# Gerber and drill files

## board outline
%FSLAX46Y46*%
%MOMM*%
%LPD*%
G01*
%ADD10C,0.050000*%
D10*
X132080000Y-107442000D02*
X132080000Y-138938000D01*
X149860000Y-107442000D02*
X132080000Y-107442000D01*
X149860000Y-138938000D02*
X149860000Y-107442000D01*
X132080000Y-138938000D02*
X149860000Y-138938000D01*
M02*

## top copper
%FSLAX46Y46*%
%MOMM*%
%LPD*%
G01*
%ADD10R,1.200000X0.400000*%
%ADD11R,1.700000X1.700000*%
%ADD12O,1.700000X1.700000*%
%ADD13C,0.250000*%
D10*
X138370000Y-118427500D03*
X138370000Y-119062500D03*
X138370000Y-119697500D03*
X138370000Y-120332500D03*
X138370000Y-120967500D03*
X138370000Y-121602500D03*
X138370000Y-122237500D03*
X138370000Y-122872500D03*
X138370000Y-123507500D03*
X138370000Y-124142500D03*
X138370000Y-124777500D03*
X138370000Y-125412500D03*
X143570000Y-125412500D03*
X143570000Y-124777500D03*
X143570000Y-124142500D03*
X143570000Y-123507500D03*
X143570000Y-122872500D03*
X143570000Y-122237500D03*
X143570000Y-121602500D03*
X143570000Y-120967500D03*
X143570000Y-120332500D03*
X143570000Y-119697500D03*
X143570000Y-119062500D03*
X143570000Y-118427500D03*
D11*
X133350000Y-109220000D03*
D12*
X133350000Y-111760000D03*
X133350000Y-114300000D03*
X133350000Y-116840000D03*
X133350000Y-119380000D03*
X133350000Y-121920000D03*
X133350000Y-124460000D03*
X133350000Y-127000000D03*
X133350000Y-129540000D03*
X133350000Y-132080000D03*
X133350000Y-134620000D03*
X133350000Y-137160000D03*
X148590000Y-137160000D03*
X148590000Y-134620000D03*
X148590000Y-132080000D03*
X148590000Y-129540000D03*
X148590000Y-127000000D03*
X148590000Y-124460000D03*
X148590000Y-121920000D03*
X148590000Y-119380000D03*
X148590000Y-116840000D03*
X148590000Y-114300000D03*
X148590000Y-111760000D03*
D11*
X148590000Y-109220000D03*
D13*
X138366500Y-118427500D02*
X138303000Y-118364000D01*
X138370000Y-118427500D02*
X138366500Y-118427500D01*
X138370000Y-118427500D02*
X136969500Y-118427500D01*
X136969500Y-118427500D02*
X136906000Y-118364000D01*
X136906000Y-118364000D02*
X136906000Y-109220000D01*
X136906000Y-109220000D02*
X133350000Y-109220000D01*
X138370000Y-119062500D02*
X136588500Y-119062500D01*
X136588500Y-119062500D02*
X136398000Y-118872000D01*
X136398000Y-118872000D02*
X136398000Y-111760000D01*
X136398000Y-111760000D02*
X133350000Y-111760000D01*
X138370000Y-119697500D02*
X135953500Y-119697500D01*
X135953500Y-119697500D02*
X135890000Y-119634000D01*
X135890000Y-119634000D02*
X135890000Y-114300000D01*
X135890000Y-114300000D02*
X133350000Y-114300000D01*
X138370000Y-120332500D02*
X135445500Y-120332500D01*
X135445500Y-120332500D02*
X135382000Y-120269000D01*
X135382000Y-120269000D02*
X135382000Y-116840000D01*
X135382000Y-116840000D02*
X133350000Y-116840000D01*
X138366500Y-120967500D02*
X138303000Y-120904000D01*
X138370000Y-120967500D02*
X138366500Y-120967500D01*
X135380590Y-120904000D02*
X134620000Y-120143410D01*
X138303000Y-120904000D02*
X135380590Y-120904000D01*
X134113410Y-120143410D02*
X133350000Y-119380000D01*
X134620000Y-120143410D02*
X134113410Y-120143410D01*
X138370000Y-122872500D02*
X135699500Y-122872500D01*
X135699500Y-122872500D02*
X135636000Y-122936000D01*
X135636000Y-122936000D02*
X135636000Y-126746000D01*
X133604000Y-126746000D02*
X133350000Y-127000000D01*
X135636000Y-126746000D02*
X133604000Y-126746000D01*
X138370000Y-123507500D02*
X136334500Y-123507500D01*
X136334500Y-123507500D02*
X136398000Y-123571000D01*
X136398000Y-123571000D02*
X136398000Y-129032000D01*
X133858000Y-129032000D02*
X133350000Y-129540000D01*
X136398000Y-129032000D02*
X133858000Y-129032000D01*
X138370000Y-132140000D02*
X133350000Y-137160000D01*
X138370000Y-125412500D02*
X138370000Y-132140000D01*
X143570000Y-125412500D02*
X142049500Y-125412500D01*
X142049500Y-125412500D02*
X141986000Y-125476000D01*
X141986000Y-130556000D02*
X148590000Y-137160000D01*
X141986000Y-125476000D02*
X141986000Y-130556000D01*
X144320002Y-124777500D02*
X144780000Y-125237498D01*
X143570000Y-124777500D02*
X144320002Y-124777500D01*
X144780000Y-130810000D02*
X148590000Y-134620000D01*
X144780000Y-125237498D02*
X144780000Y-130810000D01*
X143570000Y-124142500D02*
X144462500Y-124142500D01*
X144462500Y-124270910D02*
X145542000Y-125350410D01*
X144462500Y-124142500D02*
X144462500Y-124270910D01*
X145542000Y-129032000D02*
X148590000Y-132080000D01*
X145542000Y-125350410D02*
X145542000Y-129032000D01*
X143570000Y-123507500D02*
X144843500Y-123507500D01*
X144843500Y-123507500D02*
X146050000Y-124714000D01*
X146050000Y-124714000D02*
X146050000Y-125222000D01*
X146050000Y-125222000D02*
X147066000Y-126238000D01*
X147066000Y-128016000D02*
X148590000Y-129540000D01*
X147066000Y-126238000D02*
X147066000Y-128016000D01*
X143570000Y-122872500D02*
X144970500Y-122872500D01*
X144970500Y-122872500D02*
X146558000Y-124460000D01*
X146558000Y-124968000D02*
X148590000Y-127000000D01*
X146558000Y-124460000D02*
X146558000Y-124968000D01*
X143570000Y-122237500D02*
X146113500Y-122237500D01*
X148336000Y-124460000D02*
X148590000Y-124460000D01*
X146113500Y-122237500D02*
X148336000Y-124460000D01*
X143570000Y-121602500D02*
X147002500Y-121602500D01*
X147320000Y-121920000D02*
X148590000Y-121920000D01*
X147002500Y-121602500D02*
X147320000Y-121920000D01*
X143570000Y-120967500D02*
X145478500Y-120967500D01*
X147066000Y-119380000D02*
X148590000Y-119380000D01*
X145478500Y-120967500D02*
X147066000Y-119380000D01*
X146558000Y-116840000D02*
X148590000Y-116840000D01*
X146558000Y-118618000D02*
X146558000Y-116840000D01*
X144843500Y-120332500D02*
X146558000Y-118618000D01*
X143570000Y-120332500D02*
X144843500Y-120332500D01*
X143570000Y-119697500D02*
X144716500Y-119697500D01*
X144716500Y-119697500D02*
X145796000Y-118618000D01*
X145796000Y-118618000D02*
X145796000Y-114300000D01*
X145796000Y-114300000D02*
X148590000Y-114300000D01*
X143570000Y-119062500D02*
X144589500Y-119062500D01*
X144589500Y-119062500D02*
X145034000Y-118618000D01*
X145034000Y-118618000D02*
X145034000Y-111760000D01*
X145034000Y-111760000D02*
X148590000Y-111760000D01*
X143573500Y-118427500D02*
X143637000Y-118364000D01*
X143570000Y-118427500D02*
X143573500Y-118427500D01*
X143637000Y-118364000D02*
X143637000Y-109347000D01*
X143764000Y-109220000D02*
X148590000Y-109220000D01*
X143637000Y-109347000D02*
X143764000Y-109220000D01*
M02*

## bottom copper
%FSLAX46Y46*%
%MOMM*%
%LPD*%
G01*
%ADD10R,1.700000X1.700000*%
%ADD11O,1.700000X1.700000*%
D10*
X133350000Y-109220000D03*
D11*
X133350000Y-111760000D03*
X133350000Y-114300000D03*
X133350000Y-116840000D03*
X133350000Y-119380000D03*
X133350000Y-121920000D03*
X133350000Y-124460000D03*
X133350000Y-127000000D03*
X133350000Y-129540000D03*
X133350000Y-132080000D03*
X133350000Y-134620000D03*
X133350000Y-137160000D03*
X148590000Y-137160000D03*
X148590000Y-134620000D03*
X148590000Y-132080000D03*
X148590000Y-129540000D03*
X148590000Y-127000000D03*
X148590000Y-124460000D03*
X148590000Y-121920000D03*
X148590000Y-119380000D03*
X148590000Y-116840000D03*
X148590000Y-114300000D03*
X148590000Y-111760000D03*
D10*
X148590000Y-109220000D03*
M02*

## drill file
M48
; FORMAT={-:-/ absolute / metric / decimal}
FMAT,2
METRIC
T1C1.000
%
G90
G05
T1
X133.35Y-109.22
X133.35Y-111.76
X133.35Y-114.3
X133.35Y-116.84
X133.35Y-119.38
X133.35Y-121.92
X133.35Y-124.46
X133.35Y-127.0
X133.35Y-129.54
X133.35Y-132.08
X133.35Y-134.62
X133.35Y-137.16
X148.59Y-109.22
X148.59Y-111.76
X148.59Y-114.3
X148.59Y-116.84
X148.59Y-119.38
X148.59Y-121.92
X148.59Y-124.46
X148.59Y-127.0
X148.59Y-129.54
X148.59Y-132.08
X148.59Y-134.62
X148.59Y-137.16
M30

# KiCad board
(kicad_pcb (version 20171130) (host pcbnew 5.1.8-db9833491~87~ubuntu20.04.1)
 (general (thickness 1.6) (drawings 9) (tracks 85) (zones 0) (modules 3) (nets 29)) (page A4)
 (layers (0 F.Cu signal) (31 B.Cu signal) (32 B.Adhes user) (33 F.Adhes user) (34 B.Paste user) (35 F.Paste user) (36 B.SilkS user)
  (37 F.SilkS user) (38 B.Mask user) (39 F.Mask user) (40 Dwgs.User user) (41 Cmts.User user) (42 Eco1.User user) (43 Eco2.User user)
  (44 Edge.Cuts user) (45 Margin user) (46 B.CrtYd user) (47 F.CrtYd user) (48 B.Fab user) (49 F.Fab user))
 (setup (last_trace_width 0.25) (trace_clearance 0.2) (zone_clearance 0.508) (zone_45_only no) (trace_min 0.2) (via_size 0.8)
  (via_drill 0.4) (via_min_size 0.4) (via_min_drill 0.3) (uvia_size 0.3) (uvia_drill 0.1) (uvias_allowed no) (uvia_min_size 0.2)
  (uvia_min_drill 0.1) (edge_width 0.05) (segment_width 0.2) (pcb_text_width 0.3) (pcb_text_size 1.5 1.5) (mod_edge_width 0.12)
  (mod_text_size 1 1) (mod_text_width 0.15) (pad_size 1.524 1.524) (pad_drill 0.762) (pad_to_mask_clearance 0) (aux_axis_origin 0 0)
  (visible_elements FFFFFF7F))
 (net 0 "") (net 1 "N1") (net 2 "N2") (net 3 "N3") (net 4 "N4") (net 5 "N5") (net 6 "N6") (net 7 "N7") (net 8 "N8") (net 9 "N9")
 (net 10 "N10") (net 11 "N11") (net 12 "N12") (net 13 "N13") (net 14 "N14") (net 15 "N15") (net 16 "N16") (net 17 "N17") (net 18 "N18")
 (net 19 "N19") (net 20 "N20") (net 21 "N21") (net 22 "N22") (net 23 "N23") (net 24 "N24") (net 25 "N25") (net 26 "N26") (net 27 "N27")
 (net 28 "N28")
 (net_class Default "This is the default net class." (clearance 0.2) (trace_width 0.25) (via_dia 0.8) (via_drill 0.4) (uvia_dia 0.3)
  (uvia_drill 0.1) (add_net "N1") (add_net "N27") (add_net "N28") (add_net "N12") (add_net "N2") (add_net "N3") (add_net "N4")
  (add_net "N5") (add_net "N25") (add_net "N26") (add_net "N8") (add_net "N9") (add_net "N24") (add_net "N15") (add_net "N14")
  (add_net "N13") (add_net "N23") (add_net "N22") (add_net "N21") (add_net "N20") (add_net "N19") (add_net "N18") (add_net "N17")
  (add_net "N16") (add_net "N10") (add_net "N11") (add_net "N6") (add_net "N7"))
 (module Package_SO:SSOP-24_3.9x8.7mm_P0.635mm (layer F.Cu) (at 140.97 121.92)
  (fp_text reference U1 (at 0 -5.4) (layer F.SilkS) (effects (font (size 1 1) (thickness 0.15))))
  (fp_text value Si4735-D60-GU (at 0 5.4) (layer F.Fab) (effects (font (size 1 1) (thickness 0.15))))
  (pad 1 smd rect (at -2.6 -3.4925) (size 1.2 0.4) (layers F.Cu F.Paste F.Mask) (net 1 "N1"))
  (pad 2 smd rect (at -2.6 -2.8575) (size 1.2 0.4) (layers F.Cu F.Paste F.Mask) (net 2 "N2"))
  (pad 3 smd rect (at -2.6 -2.2225) (size 1.2 0.4) (layers F.Cu F.Paste F.Mask) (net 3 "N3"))
  (pad 4 smd rect (at -2.6 -1.5875) (size 1.2 0.4) (layers F.Cu F.Paste F.Mask) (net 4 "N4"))
  (pad 5 smd rect (at -2.6 -0.9525) (size 1.2 0.4) (layers F.Cu F.Paste F.Mask) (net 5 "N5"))
  (pad 6 smd rect (at -2.6 -0.3175) (size 1.2 0.4) (layers F.Cu F.Paste F.Mask) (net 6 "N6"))
  (pad 7 smd rect (at -2.6 0.3175) (size 1.2 0.4) (layers F.Cu F.Paste F.Mask) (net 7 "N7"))
  (pad 8 smd rect (at -2.6 0.9525) (size 1.2 0.4) (layers F.Cu F.Paste F.Mask) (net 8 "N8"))
  (pad 9 smd rect (at -2.6 1.5875) (size 1.2 0.4) (layers F.Cu F.Paste F.Mask) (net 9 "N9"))
  (pad 10 smd rect (at -2.6 2.2225) (size 1.2 0.4) (layers F.Cu F.Paste F.Mask) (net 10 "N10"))
  (pad 11 smd rect (at -2.6 2.8575) (size 1.2 0.4) (layers F.Cu F.Paste F.Mask) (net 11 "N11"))
  (pad 12 smd rect (at -2.6 3.4925) (size 1.2 0.4) (layers F.Cu F.Paste F.Mask) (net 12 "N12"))
  (pad 13 smd rect (at 2.6 3.4925) (size 1.2 0.4) (layers F.Cu F.Paste F.Mask) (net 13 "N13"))
  (pad 14 smd rect (at 2.6 2.8575) (size 1.2 0.4) (layers F.Cu F.Paste F.Mask) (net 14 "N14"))
  (pad 15 smd rect (at 2.6 2.2225) (size 1.2 0.4) (layers F.Cu F.Paste F.Mask) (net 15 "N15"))
  (pad 16 smd rect (at 2.6 1.5875) (size 1.2 0.4) (layers F.Cu F.Paste F.Mask) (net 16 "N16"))
  (pad 17 smd rect (at 2.6 0.9525) (size 1.2 0.4) (layers F.Cu F.Paste F.Mask) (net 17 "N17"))
  (pad 18 smd rect (at 2.6 0.3175) (size 1.2 0.4) (layers F.Cu F.Paste F.Mask) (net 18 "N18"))
  (pad 19 smd rect (at 2.6 -0.3175) (size 1.2 0.4) (layers F.Cu F.Paste F.Mask) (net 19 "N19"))
  (pad 20 smd rect (at 2.6 -0.9525) (size 1.2 0.4) (layers F.Cu F.Paste F.Mask) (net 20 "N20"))
  (pad 21 smd rect (at 2.6 -1.5875) (size 1.2 0.4) (layers F.Cu F.Paste F.Mask) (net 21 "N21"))
  (pad 22 smd rect (at 2.6 -2.2225) (size 1.2 0.4) (layers F.Cu F.Paste F.Mask) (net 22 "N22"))
  (pad 23 smd rect (at 2.6 -2.8575) (size 1.2 0.4) (layers F.Cu F.Paste F.Mask) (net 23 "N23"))
  (pad 24 smd rect (at 2.6 -3.4925) (size 1.2 0.4) (layers F.Cu F.Paste F.Mask) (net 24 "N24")))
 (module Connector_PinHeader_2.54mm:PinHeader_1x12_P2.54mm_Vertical (layer F.Cu) (at 133.35 109.22)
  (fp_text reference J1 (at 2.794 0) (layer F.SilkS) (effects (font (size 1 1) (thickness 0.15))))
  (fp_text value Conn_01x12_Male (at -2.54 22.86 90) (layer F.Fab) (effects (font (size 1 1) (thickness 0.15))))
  (pad 1 thru_hole rect (at 0 0) (size 1.7 1.7) (drill 1) (layers *.Cu *.Mask) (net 1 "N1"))
  (pad 2 thru_hole oval (at 0 2.54) (size 1.7 1.7) (drill 1) (layers *.Cu *.Mask) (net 2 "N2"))
  (pad 3 thru_hole oval (at 0 5.08) (size 1.7 1.7) (drill 1) (layers *.Cu *.Mask) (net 3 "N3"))
  (pad 4 thru_hole oval (at 0 7.62) (size 1.7 1.7) (drill 1) (layers *.Cu *.Mask) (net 4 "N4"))
  (pad 5 thru_hole oval (at 0 10.16) (size 1.7 1.7) (drill 1) (layers *.Cu *.Mask) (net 5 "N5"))
  (pad 6 thru_hole oval (at 0 12.7) (size 1.7 1.7) (drill 1) (layers *.Cu *.Mask) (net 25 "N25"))
  (pad 7 thru_hole oval (at 0 15.24) (size 1.7 1.7) (drill 1) (layers *.Cu *.Mask) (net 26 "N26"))
  (pad 8 thru_hole oval (at 0 17.78) (size 1.7 1.7) (drill 1) (layers *.Cu *.Mask) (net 8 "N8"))
  (pad 9 thru_hole oval (at 0 20.32) (size 1.7 1.7) (drill 1) (layers *.Cu *.Mask) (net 9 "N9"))
  (pad 10 thru_hole oval (at 0 22.86) (size 1.7 1.7) (drill 1) (layers *.Cu *.Mask) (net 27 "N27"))
  (pad 11 thru_hole oval (at 0 25.4) (size 1.7 1.7) (drill 1) (layers *.Cu *.Mask) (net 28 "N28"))
  (pad 12 thru_hole oval (at 0 27.94) (size 1.7 1.7) (drill 1) (layers *.Cu *.Mask) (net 12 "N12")))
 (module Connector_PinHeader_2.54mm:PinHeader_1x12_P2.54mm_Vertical (layer F.Cu) (at 148.59 109.22)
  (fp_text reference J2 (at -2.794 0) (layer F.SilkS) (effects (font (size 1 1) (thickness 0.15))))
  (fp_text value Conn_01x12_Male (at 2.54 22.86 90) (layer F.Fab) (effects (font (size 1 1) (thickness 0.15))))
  (pad 12 thru_hole oval (at 0 27.94) (size 1.7 1.7) (drill 1) (layers *.Cu *.Mask) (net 13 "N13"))
  (pad 11 thru_hole oval (at 0 25.4) (size 1.7 1.7) (drill 1) (layers *.Cu *.Mask) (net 14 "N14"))
  (pad 10 thru_hole oval (at 0 22.86) (size 1.7 1.7) (drill 1) (layers *.Cu *.Mask) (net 15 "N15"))
  (pad 9 thru_hole oval (at 0 20.32) (size 1.7 1.7) (drill 1) (layers *.Cu *.Mask) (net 16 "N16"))
  (pad 8 thru_hole oval (at 0 17.78) (size 1.7 1.7) (drill 1) (layers *.Cu *.Mask) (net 17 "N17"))
  (pad 7 thru_hole oval (at 0 15.24) (size 1.7 1.7) (drill 1) (layers *.Cu *.Mask) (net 18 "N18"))
  (pad 6 thru_hole oval (at 0 12.7) (size 1.7 1.7) (drill 1) (layers *.Cu *.Mask) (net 19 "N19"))
  (pad 5 thru_hole oval (at 0 10.16) (size 1.7 1.7) (drill 1) (layers *.Cu *.Mask) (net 20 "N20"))
  (pad 4 thru_hole oval (at 0 7.62) (size 1.7 1.7) (drill 1) (layers *.Cu *.Mask) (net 21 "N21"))
  (pad 3 thru_hole oval (at 0 5.08) (size 1.7 1.7) (drill 1) (layers *.Cu *.Mask) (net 22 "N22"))
  (pad 2 thru_hole oval (at 0 2.54) (size 1.7 1.7) (drill 1) (layers *.Cu *.Mask) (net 23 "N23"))
  (pad 1 thru_hole rect (at 0 0) (size 1.7 1.7) (drill 1) (layers *.Cu *.Mask) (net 24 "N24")))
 (gr_line (start 132.08 107.442) (end 132.08 138.938) (layer Edge.Cuts) (width 0.05))
 (gr_line (start 149.86 107.442) (end 132.08 107.442) (layer Edge.Cuts) (width 0.05))
 (gr_line (start 149.86 138.938) (end 149.86 107.442) (layer Edge.Cuts) (width 0.05))
 (gr_line (start 132.08 138.938) (end 149.86 138.938) (layer Edge.Cuts) (width 0.05))
 (segment (start 138.3665 118.4275) (end 138.303 118.364) (width 0.25) (layer F.Cu) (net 1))
 (segment (start 138.37 118.4275) (end 138.3665 118.4275) (width 0.25) (layer F.Cu) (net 1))
 (segment (start 138.37 118.4275) (end 136.9695 118.4275) (width 0.25) (layer F.Cu) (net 1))
 (segment (start 136.9695 118.4275) (end 136.906 118.364) (width 0.25) (layer F.Cu) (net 1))
 (segment (start 136.906 118.364) (end 136.906 109.22) (width 0.25) (layer F.Cu) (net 1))
 (segment (start 136.906 109.22) (end 133.35 109.22) (width 0.25) (layer F.Cu) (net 1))
 (segment (start 138.37 119.0625) (end 136.5885 119.0625) (width 0.25) (layer F.Cu) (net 2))
 (segment (start 136.5885 119.0625) (end 136.398 118.872) (width 0.25) (layer F.Cu) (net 2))
 (segment (start 136.398 118.872) (end 136.398 111.76) (width 0.25) (layer F.Cu) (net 2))
 (segment (start 136.398 111.76) (end 133.35 111.76) (width 0.25) (layer F.Cu) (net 2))
 (segment (start 138.37 119.6975) (end 135.9535 119.6975) (width 0.25) (layer F.Cu) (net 3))
 (segment (start 135.9535 119.6975) (end 135.89 119.634) (width 0.25) (layer F.Cu) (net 3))
 (segment (start 135.89 119.634) (end 135.89 114.3) (width 0.25) (layer F.Cu) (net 3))
 (segment (start 135.89 114.3) (end 133.35 114.3) (width 0.25) (layer F.Cu) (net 3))
 (segment (start 138.37 120.3325) (end 135.4455 120.3325) (width 0.25) (layer F.Cu) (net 4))
 (segment (start 135.4455 120.3325) (end 135.382 120.269) (width 0.25) (layer F.Cu) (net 4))
 (segment (start 135.382 120.269) (end 135.382 116.84) (width 0.25) (layer F.Cu) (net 4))
 (segment (start 135.382 116.84) (end 133.35 116.84) (width 0.25) (layer F.Cu) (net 4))
 (segment (start 138.3665 120.9675) (end 138.303 120.904) (width 0.25) (layer F.Cu) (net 5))
 (segment (start 138.37 120.9675) (end 138.3665 120.9675) (width 0.25) (layer F.Cu) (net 5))
 (segment (start 135.38059 120.904) (end 134.62 120.14341) (width 0.25) (layer F.Cu) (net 5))
 (segment (start 138.303 120.904) (end 135.38059 120.904) (width 0.25) (layer F.Cu) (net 5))
 (segment (start 134.11341 120.14341) (end 133.35 119.38) (width 0.25) (layer F.Cu) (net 5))
 (segment (start 134.62 120.14341) (end 134.11341 120.14341) (width 0.25) (layer F.Cu) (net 5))
 (segment (start 138.37 122.8725) (end 135.6995 122.8725) (width 0.25) (layer F.Cu) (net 8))
 (segment (start 135.6995 122.8725) (end 135.636 122.936) (width 0.25) (layer F.Cu) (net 8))
 (segment (start 135.636 122.936) (end 135.636 126.746) (width 0.25) (layer F.Cu) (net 8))
 (segment (start 133.604 126.746) (end 133.35 127) (width 0.25) (layer F.Cu) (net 8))
 (segment (start 135.636 126.746) (end 133.604 126.746) (width 0.25) (layer F.Cu) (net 8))
 (segment (start 138.37 123.5075) (end 136.3345 123.5075) (width 0.25) (layer F.Cu) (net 9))
 (segment (start 136.3345 123.5075) (end 136.398 123.571) (width 0.25) (layer F.Cu) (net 9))
 (segment (start 136.398 123.571) (end 136.398 129.032) (width 0.25) (layer F.Cu) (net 9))
 (segment (start 133.858 129.032) (end 133.35 129.54) (width 0.25) (layer F.Cu) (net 9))
 (segment (start 136.398 129.032) (end 133.858 129.032) (width 0.25) (layer F.Cu) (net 9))
 (segment (start 138.37 132.14) (end 133.35 137.16) (width 0.25) (layer F.Cu) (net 12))
 (segment (start 138.37 125.4125) (end 138.37 132.14) (width 0.25) (layer F.Cu) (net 12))
 (segment (start 143.57 125.4125) (end 142.0495 125.4125) (width 0.25) (layer F.Cu) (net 13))
 (segment (start 142.0495 125.4125) (end 141.986 125.476) (width 0.25) (layer F.Cu) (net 13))
 (segment (start 141.986 130.556) (end 148.59 137.16) (width 0.25) (layer F.Cu) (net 13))
 (segment (start 141.986 125.476) (end 141.986 130.556) (width 0.25) (layer F.Cu) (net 13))
 (segment (start 144.320002 124.7775) (end 144.78 125.237498) (width 0.25) (layer F.Cu) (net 14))
 (segment (start 143.57 124.7775) (end 144.320002 124.7775) (width 0.25) (layer F.Cu) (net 14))
 (segment (start 144.78 130.81) (end 148.59 134.62) (width 0.25) (layer F.Cu) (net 14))
 (segment (start 144.78 125.237498) (end 144.78 130.81) (width 0.25) (layer F.Cu) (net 14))
 (segment (start 143.57 124.1425) (end 144.4625 124.1425) (width 0.25) (layer F.Cu) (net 15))
 (segment (start 144.4625 124.27091) (end 145.542 125.35041) (width 0.25) (layer F.Cu) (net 15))
 (segment (start 144.4625 124.1425) (end 144.4625 124.27091) (width 0.25) (layer F.Cu) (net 15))
 (segment (start 145.542 129.032) (end 148.59 132.08) (width 0.25) (layer F.Cu) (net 15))
 (segment (start 145.542 125.35041) (end 145.542 129.032) (width 0.25) (layer F.Cu) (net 15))
 (segment (start 143.57 123.5075) (end 144.8435 123.5075) (width 0.25) (layer F.Cu) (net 16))
 (segment (start 144.8435 123.5075) (end 146.05 124.714) (width 0.25) (layer F.Cu) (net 16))
 (segment (start 146.05 124.714) (end 146.05 125.222) (width 0.25) (layer F.Cu) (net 16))
 (segment (start 146.05 125.222) (end 147.066 126.238) (width 0.25) (layer F.Cu) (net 16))
 (segment (start 147.066 128.016) (end 148.59 129.54) (width 0.25) (layer F.Cu) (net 16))
 (segment (start 147.066 126.238) (end 147.066 128.016) (width 0.25) (layer F.Cu) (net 16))
 (segment (start 143.57 122.8725) (end 144.9705 122.8725) (width 0.25) (layer F.Cu) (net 17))
 (segment (start 144.9705 122.8725) (end 146.558 124.46) (width 0.25) (layer F.Cu) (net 17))
 (segment (start 146.558 124.968) (end 148.59 127) (width 0.25) (layer F.Cu) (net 17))
 (segment (start 146.558 124.46) (end 146.558 124.968) (width 0.25) (layer F.Cu) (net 17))
 (segment (start 143.57 122.2375) (end 146.1135 122.2375) (width 0.25) (layer F.Cu) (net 18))
 (segment (start 148.336 124.46) (end 148.59 124.46) (width 0.25) (layer F.Cu) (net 18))
 (segment (start 146.1135 122.2375) (end 148.336 124.46) (width 0.25) (layer F.Cu) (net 18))
 (segment (start 143.57 121.6025) (end 147.0025 121.6025) (width 0.25) (layer F.Cu) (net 19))
 (segment (start 147.32 121.92) (end 148.59 121.92) (width 0.25) (layer F.Cu) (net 19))
 (segment (start 147.0025 121.6025) (end 147.32 121.92) (width 0.25) (layer F.Cu) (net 19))
 (segment (start 143.57 120.9675) (end 145.4785 120.9675) (width 0.25) (layer F.Cu) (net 20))
 (segment (start 147.066 119.38) (end 148.59 119.38) (width 0.25) (layer F.Cu) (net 20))
 (segment (start 145.4785 120.9675) (end 147.066 119.38) (width 0.25) (layer F.Cu) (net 20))
 (segment (start 146.558 116.84) (end 148.59 116.84) (width 0.25) (layer F.Cu) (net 21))
 (segment (start 146.558 118.618) (end 146.558 116.84) (width 0.25) (layer F.Cu) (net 21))
 (segment (start 144.8435 120.3325) (end 146.558 118.618) (width 0.25) (layer F.Cu) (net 21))
 (segment (start 143.57 120.3325) (end 144.8435 120.3325) (width 0.25) (layer F.Cu) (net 21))
 (segment (start 143.57 119.6975) (end 144.7165 119.6975) (width 0.25) (layer F.Cu) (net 22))
 (segment (start 144.7165 119.6975) (end 145.796 118.618) (width 0.25) (layer F.Cu) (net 22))
 (segment (start 145.796 118.618) (end 145.796 114.3) (width 0.25) (layer F.Cu) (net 22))
 (segment (start 145.796 114.3) (end 148.59 114.3) (width 0.25) (layer F.Cu) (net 22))
 (segment (start 143.57 119.0625) (end 144.5895 119.0625) (width 0.25) (layer F.Cu) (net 23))
 (segment (start 144.5895 119.0625) (end 145.034 118.618) (width 0.25) (layer F.Cu) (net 23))
 (segment (start 145.034 118.618) (end 145.034 111.76) (width 0.25) (layer F.Cu) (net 23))
 (segment (start 145.034 111.76) (end 148.59 111.76) (width 0.25) (layer F.Cu) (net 23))
 (segment (start 143.5735 118.4275) (end 143.637 118.364) (width 0.25) (layer F.Cu) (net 24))
 (segment (start 143.57 118.4275) (end 143.5735 118.4275) (width 0.25) (layer F.Cu) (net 24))
 (segment (start 143.637 118.364) (end 143.637 109.347) (width 0.25) (layer F.Cu) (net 24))
 (segment (start 143.764 109.22) (end 148.59 109.22) (width 0.25) (layer F.Cu) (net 24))
 (segment (start 143.637 109.347) (end 143.764 109.22) (width 0.25) (layer F.Cu) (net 24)))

